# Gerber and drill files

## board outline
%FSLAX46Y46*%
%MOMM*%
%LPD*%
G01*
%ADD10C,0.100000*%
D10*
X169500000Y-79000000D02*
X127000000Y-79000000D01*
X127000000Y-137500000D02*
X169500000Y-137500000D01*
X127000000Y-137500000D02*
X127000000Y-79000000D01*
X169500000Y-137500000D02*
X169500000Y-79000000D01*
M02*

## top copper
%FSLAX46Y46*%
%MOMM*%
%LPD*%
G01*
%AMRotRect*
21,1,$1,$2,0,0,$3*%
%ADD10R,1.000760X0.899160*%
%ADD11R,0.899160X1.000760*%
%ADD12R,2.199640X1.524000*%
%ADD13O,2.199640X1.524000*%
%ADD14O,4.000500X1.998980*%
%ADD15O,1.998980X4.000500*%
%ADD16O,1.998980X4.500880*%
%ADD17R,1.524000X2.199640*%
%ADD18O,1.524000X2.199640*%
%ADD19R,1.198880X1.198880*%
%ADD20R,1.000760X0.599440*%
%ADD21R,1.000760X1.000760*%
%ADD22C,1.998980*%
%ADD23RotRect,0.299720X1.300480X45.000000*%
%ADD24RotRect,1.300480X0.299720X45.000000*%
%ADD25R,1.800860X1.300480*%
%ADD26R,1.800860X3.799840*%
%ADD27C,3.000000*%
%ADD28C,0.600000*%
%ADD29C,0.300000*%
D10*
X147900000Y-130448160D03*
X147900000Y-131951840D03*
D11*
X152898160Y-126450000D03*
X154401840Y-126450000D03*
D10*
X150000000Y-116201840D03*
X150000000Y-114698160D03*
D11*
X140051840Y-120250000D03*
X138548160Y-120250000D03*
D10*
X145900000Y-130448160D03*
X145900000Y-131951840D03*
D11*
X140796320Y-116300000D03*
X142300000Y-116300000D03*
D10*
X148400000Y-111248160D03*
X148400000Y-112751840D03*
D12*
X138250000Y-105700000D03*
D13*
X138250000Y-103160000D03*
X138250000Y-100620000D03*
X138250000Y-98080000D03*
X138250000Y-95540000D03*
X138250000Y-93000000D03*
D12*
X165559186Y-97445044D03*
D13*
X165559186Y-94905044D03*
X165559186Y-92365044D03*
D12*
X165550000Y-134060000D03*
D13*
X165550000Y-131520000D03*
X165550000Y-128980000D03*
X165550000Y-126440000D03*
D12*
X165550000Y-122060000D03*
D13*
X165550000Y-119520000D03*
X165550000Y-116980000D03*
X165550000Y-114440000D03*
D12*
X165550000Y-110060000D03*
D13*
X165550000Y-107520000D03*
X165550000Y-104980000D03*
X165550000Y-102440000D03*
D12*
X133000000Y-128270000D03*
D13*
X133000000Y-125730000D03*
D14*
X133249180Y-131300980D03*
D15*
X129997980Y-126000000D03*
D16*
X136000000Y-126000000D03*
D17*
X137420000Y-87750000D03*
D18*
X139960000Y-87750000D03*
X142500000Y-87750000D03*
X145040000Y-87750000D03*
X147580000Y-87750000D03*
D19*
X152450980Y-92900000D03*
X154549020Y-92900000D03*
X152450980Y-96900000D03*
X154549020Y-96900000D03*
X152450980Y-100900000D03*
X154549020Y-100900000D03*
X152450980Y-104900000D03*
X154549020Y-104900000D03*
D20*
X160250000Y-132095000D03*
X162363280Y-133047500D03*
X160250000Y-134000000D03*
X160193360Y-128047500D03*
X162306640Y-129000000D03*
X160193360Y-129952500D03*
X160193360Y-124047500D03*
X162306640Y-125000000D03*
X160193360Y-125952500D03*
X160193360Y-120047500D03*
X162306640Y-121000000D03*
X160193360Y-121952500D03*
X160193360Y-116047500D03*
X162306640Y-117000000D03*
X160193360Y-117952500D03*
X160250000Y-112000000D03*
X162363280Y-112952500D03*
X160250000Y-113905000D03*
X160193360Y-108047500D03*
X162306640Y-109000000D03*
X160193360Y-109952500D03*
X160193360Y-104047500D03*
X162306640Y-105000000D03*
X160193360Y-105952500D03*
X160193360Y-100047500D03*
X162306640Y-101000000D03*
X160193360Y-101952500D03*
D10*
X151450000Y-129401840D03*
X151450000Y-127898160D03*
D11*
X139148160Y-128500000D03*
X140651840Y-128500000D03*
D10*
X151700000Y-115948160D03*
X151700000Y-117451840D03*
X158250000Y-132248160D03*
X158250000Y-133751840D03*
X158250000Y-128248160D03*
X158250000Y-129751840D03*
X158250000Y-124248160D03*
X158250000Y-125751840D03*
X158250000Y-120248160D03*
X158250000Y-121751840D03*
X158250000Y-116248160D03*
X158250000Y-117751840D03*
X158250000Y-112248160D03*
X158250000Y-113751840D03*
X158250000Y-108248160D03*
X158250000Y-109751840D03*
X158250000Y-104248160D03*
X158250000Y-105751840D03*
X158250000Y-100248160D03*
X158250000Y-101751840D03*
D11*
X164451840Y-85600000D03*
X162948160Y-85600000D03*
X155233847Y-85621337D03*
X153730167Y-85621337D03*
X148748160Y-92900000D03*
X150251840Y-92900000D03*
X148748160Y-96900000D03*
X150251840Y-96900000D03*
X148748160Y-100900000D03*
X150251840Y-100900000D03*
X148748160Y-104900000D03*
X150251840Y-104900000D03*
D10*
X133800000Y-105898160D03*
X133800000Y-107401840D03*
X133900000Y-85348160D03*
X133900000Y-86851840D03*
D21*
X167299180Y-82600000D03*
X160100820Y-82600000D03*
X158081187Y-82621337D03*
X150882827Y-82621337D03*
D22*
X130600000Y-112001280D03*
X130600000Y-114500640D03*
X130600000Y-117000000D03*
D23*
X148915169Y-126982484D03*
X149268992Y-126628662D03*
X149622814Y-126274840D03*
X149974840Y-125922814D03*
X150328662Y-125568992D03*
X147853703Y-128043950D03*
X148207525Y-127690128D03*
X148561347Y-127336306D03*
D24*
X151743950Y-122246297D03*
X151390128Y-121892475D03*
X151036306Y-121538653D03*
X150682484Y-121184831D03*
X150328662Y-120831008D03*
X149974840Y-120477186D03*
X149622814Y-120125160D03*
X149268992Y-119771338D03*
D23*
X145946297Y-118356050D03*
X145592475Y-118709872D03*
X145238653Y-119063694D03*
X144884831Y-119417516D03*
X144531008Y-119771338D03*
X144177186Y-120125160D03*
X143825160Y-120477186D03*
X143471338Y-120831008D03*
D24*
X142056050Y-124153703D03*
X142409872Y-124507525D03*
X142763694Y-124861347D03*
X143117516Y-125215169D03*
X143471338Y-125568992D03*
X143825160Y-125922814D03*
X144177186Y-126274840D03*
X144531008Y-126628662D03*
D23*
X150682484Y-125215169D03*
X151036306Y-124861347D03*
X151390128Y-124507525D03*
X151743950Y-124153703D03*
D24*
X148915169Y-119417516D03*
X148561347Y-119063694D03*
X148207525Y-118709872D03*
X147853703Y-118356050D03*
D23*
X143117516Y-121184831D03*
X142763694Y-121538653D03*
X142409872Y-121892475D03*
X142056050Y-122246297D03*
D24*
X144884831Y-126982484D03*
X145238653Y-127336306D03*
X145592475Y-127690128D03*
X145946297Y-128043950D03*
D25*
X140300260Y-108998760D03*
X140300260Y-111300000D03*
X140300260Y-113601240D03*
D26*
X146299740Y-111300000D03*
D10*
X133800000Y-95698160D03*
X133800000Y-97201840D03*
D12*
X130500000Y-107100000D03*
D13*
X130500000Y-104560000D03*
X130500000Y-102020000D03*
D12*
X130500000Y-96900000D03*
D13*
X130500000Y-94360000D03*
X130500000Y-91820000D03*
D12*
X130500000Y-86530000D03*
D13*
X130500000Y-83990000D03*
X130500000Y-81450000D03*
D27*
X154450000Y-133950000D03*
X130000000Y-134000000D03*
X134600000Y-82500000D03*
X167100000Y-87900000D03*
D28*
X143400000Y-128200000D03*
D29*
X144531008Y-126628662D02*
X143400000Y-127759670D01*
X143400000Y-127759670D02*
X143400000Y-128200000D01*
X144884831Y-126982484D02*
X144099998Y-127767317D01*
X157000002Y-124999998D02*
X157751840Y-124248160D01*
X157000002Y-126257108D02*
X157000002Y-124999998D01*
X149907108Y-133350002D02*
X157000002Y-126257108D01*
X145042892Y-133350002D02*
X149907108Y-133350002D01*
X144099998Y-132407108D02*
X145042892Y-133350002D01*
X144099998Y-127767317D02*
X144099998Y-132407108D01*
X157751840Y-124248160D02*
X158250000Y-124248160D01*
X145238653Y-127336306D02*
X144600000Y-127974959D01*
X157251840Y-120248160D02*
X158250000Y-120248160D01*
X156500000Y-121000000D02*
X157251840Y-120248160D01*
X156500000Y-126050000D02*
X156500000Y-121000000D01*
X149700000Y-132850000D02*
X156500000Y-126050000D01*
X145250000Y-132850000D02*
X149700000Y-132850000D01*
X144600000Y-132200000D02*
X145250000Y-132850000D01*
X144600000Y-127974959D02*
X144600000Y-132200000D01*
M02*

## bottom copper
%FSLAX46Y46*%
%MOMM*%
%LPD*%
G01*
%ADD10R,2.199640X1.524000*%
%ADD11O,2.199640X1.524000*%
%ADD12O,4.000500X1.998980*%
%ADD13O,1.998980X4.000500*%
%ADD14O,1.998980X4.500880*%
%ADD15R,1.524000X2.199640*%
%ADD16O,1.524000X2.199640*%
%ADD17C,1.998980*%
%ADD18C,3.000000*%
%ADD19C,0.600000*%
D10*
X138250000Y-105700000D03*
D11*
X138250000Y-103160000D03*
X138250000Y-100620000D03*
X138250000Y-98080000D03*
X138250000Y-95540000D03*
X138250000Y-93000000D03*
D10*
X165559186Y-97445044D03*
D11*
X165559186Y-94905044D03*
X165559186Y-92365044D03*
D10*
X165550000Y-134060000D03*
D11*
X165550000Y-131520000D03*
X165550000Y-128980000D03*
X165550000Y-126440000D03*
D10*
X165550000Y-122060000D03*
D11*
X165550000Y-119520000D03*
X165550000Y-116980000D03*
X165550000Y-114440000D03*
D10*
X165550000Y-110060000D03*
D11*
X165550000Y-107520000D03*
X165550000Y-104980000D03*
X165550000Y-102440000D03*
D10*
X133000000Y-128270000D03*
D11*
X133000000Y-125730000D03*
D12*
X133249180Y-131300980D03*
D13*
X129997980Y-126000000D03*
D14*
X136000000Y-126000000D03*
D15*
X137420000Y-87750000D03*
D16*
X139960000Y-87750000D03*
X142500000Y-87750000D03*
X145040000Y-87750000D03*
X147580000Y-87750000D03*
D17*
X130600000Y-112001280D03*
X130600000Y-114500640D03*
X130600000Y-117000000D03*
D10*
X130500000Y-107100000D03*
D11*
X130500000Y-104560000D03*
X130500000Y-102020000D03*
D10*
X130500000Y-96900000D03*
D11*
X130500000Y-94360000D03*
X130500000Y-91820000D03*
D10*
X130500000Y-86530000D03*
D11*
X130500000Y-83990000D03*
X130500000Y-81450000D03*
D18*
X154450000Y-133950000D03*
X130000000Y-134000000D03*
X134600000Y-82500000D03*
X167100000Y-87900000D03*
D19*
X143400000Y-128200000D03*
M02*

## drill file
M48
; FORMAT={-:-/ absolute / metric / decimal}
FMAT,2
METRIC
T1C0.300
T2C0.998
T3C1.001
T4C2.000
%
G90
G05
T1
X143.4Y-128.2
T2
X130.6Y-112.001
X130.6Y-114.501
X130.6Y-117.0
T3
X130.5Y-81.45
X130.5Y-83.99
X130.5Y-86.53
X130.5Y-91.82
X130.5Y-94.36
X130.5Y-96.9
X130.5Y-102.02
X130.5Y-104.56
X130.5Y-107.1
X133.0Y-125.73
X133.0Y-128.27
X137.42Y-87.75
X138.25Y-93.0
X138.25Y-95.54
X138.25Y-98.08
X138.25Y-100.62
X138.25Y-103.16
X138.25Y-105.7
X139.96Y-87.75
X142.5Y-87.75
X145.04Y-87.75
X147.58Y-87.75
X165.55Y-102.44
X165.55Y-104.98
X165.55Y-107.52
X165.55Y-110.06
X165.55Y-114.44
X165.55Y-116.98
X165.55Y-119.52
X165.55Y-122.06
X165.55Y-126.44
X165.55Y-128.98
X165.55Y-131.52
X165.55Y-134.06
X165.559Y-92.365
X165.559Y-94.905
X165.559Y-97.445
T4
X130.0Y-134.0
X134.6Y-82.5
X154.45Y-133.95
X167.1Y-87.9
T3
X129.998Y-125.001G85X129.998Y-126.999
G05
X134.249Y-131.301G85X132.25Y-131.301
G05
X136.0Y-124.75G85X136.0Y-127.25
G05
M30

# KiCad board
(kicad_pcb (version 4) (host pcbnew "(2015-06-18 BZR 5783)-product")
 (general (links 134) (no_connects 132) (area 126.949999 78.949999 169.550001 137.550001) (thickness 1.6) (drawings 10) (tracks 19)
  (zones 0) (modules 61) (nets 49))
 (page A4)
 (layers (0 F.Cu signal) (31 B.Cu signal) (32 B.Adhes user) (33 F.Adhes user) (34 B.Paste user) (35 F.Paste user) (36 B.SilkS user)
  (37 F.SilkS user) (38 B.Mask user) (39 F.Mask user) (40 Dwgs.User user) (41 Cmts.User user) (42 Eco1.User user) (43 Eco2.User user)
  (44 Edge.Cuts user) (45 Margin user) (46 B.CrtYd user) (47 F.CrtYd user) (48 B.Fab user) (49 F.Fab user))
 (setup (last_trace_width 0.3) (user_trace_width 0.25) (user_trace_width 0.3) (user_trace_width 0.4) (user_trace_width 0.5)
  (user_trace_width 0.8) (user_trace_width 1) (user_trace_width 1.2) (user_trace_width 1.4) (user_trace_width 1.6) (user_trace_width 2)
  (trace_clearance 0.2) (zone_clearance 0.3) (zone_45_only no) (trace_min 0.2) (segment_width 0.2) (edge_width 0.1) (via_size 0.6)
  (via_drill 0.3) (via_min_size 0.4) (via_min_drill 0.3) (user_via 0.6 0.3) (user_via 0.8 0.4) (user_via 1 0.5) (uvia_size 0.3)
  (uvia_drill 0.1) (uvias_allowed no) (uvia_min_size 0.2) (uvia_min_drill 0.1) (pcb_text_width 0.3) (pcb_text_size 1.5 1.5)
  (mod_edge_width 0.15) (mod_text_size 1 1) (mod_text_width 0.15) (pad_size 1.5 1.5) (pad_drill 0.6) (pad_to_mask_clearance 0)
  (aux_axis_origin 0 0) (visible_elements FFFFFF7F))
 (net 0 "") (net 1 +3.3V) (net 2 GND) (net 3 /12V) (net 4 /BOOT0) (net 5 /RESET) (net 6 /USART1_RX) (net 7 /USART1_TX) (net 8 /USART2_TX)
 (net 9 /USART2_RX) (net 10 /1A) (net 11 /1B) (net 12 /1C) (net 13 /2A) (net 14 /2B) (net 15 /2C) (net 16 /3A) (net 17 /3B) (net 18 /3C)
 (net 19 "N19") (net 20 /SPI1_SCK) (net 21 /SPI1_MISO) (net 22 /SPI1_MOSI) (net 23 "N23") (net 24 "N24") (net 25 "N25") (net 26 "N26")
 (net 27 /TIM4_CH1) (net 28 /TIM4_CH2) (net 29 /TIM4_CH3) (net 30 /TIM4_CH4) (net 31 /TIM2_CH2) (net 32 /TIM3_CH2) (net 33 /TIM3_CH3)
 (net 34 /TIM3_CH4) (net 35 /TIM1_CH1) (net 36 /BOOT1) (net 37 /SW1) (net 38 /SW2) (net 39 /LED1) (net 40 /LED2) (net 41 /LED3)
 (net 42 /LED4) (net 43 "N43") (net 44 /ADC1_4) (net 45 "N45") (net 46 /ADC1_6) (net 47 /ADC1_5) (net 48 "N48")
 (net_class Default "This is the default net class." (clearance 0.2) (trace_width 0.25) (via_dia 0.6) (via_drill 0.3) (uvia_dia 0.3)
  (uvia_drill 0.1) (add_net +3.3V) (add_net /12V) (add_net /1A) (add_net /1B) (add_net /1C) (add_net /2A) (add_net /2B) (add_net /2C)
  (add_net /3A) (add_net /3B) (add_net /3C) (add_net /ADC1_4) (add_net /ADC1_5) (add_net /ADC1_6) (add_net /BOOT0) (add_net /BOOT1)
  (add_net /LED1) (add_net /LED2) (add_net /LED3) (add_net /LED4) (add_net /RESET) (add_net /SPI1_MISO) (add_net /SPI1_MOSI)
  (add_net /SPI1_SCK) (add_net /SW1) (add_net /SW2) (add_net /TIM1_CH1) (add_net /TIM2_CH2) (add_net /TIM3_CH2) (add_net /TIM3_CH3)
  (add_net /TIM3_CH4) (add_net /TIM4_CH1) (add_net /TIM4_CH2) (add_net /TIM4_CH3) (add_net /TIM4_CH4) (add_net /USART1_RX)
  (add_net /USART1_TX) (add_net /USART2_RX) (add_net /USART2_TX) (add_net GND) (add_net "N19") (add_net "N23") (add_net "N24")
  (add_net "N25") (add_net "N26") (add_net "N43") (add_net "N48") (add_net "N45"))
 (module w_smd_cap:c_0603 (layer F.Cu) (at 147.9 131.2 90)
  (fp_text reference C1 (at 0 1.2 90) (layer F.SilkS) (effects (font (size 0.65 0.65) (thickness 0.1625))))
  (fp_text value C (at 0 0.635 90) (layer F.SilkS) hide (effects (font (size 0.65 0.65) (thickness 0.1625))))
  (pad 1 smd rect (at 0.75184 0 90) (size 0.89916 1.00076) (layers F.Cu F.Paste F.Mask) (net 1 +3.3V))
  (pad 2 smd rect (at -0.75184 0 90) (size 0.89916 1.00076) (layers F.Cu F.Paste F.Mask) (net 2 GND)))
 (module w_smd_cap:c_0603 (layer F.Cu) (at 153.65 126.45 180)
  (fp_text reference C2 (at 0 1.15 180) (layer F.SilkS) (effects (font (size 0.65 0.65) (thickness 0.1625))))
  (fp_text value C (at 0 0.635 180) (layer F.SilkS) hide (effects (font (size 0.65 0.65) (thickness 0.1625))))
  (pad 1 smd rect (at 0.75184 0 180) (size 0.89916 1.00076) (layers F.Cu F.Paste F.Mask) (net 1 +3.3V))
  (pad 2 smd rect (at -0.75184 0 180) (size 0.89916 1.00076) (layers F.Cu F.Paste F.Mask) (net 2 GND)))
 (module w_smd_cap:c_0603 (layer F.Cu) (at 150 115.45 270)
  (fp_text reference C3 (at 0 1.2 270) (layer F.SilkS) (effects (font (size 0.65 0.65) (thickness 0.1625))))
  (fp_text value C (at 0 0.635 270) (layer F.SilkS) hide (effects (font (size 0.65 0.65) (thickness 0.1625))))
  (pad 1 smd rect (at 0.75184 0 270) (size 0.89916 1.00076) (layers F.Cu F.Paste F.Mask) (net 1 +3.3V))
  (pad 2 smd rect (at -0.75184 0 270) (size 0.89916 1.00076) (layers F.Cu F.Paste F.Mask) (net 2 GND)))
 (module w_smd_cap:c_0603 (layer F.Cu) (at 139.3 120.25)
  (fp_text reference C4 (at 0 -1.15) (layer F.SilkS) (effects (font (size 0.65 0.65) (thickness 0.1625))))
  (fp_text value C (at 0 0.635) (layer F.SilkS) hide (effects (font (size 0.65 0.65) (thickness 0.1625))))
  (pad 1 smd rect (at 0.75184 0) (size 0.89916 1.00076) (layers F.Cu F.Paste F.Mask) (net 1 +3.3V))
  (pad 2 smd rect (at -0.75184 0) (size 0.89916 1.00076) (layers F.Cu F.Paste F.Mask) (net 2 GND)))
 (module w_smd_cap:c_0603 (layer F.Cu) (at 145.9 131.2 90)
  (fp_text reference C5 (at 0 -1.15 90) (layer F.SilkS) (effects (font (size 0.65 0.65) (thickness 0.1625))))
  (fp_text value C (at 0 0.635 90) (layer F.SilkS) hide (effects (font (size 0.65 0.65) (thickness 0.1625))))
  (pad 1 smd rect (at 0.75184 0 90) (size 0.89916 1.00076) (layers F.Cu F.Paste F.Mask) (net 1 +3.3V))
  (pad 2 smd rect (at -0.75184 0 90) (size 0.89916 1.00076) (layers F.Cu F.Paste F.Mask) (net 2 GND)))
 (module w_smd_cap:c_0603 (layer F.Cu) (at 141.54816 116.3 180)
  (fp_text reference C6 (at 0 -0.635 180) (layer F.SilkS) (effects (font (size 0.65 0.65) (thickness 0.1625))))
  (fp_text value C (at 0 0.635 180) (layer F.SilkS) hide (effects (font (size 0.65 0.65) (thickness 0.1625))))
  (pad 1 smd rect (at 0.75184 0 180) (size 0.89916 1.00076) (layers F.Cu F.Paste F.Mask) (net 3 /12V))
  (pad 2 smd rect (at -0.75184 0 180) (size 0.89916 1.00076) (layers F.Cu F.Paste F.Mask) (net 2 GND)))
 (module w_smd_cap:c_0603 (layer F.Cu) (at 148.4 112 90)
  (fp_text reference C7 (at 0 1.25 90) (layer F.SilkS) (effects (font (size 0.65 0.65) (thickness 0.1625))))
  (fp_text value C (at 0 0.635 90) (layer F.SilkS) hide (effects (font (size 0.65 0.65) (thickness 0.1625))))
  (pad 1 smd rect (at 0.75184 0 90) (size 0.89916 1.00076) (layers F.Cu F.Paste F.Mask) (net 1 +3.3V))
  (pad 2 smd rect (at -0.75184 0 90) (size 0.89916 1.00076) (layers F.Cu F.Paste F.Mask) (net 2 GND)))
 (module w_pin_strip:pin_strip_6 (layer F.Cu) (at 138.25 99.35 90)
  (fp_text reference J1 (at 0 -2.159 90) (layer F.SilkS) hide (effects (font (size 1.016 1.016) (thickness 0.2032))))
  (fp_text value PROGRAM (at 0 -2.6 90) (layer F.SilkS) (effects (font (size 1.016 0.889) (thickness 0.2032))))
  (pad 1 thru_hole rect (at -6.35 0 90) (size 1.524 2.19964) (drill 1.00076) (layers *.Cu *.Mask F.SilkS) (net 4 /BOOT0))
  (pad 2 thru_hole oval (at -3.81 0 90) (size 1.524 2.19964) (drill 1.00076) (layers *.Cu *.Mask F.SilkS) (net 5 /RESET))
  (pad 3 thru_hole oval (at -1.27 0 90) (size 1.524 2.19964) (drill 1.00076) (layers *.Cu *.Mask F.SilkS) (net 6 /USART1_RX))
  (pad 4 thru_hole oval (at 1.27 0 90) (size 1.524 2.19964) (drill 1.00076) (layers *.Cu *.Mask F.SilkS) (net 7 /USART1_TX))
  (pad 5 thru_hole oval (at 3.81 0 90) (size 1.524 2.19964) (drill 1.00076) (layers *.Cu *.Mask F.SilkS) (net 2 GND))
  (pad 6 thru_hole oval (at 6.35 0 90) (size 1.524 2.19964) (drill 1.00076) (layers *.Cu *.Mask F.SilkS) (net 1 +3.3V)))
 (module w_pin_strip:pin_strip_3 (layer F.Cu) (at 165.559186 94.905044 90)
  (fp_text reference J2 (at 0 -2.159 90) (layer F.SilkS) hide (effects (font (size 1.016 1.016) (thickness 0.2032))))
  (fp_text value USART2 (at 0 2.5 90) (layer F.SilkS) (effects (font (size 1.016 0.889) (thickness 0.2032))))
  (pad 1 thru_hole rect (at -2.54 0 90) (size 1.524 2.19964) (drill 1.00076) (layers *.Cu *.Mask F.SilkS) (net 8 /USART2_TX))
  (pad 2 thru_hole oval (at 0 0 90) (size 1.524 2.19964) (drill 1.00076) (layers *.Cu *.Mask F.SilkS) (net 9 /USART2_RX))
  (pad 3 thru_hole oval (at 2.54 0 90) (size 1.524 2.19964) (drill 1.00076) (layers *.Cu *.Mask F.SilkS) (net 2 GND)))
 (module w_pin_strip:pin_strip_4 (layer F.Cu) (at 165.55 130.25 90)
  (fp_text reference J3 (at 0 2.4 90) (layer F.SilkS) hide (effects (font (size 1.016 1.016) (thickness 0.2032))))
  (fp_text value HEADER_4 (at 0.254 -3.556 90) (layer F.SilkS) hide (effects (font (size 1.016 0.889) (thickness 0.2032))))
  (pad 1 thru_hole rect (at -3.81 0 90) (size 1.524 2.19964) (drill 1.00076) (layers *.Cu *.Mask F.SilkS) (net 3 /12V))
  (pad 2 thru_hole oval (at -1.27 0 90) (size 1.524 2.19964) (drill 1.00076) (layers *.Cu *.Mask F.SilkS) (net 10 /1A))
  (pad 3 thru_hole oval (at 1.27 0 90) (size 1.524 2.19964) (drill 1.00076) (layers *.Cu *.Mask F.SilkS) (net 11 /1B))
  (pad 4 thru_hole oval (at 3.81 0 90) (size 1.524 2.19964) (drill 1.00076) (layers *.Cu *.Mask F.SilkS) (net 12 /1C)))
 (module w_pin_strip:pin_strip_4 (layer F.Cu) (at 165.55 118.25 90)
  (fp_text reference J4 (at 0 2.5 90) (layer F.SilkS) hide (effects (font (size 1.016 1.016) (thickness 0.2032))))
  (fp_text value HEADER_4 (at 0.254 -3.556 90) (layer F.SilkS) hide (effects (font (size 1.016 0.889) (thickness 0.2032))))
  (pad 1 thru_hole rect (at -3.81 0 90) (size 1.524 2.19964) (drill 1.00076) (layers *.Cu *.Mask F.SilkS) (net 3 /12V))
  (pad 2 thru_hole oval (at -1.27 0 90) (size 1.524 2.19964) (drill 1.00076) (layers *.Cu *.Mask F.SilkS) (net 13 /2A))
  (pad 3 thru_hole oval (at 1.27 0 90) (size 1.524 2.19964) (drill 1.00076) (layers *.Cu *.Mask F.SilkS) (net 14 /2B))
  (pad 4 thru_hole oval (at 3.81 0 90) (size 1.524 2.19964) (drill 1.00076) (layers *.Cu *.Mask F.SilkS) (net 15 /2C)))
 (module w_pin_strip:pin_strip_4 (layer F.Cu) (at 165.55 106.25 90)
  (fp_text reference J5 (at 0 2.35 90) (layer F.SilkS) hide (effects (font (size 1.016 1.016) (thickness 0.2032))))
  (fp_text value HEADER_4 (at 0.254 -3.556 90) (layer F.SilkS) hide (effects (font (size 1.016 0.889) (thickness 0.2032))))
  (pad 1 thru_hole rect (at -3.81 0 90) (size 1.524 2.19964) (drill 1.00076) (layers *.Cu *.Mask F.SilkS) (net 3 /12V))
  (pad 2 thru_hole oval (at -1.27 0 90) (size 1.524 2.19964) (drill 1.00076) (layers *.Cu *.Mask F.SilkS) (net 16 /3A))
  (pad 3 thru_hole oval (at 1.27 0 90) (size 1.524 2.19964) (drill 1.00076) (layers *.Cu *.Mask F.SilkS) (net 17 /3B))
  (pad 4 thru_hole oval (at 3.81 0 90) (size 1.524 2.19964) (drill 1.00076) (layers *.Cu *.Mask F.SilkS) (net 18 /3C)))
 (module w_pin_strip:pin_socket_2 (layer F.Cu) (at 133 127 90)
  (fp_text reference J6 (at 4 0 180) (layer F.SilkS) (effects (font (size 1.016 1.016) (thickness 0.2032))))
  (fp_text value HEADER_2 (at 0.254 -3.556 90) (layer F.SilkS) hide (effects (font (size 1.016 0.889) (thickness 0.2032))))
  (pad 1 thru_hole rect (at -1.27 0 90) (size 1.524 2.19964) (drill 1.00076) (layers *.Cu *.Mask F.SilkS) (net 3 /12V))
  (pad 2 thru_hole oval (at 1.27 0 90) (size 1.524 2.19964) (drill 1.00076) (layers *.Cu *.Mask F.SilkS) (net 2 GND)))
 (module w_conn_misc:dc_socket (layer F.Cu) (at 129.74906 126 270)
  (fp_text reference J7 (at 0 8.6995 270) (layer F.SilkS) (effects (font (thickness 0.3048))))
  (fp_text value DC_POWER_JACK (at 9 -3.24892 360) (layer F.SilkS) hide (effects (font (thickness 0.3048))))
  (pad 1 thru_hole oval (at 5.30098 -3.50012 270) (size 1.99898 4.0005) (drill oval 1.00076 2.99974) (layers *.Cu *.Mask F.SilkS)
   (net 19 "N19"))
  (pad 2 thru_hole oval (at 0 -0.24892 270) (size 4.0005 1.99898) (drill oval 2.99974 1.00076) (layers *.Cu *.Mask F.SilkS) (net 2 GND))
  (pad 3 thru_hole oval (at 0 -6.25094 270) (size 4.50088 1.99898) (drill oval 3.50012 1.00076) (layers *.Cu *.Mask F.SilkS) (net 2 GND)))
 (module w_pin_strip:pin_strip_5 (layer F.Cu) (at 142.5 87.75)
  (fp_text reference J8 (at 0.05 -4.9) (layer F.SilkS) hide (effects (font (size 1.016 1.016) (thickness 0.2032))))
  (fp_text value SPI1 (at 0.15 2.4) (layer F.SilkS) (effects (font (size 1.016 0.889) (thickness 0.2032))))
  (pad 1 thru_hole rect (at -5.08 0) (size 1.524 2.19964) (drill 1.00076) (layers *.Cu *.Mask F.SilkS) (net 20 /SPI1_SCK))
  (pad 2 thru_hole oval (at -2.54 0) (size 1.524 2.19964) (drill 1.00076) (layers *.Cu *.Mask F.SilkS) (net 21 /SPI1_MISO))
  (pad 3 thru_hole oval (at 0 0) (size 1.524 2.19964) (drill 1.00076) (layers *.Cu *.Mask F.SilkS) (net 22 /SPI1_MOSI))
  (pad 4 thru_hole oval (at 2.54 0) (size 1.524 2.19964) (drill 1.00076) (layers *.Cu *.Mask F.SilkS) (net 2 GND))
  (pad 5 thru_hole oval (at 5.08 0) (size 1.524 2.19964) (drill 1.00076) (layers *.Cu *.Mask F.SilkS) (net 1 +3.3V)))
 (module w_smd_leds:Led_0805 (layer F.Cu) (at 153.5 92.9)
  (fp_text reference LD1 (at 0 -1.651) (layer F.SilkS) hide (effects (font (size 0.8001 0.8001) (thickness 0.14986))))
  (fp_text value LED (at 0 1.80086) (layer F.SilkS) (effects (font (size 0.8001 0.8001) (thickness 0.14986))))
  (pad 1 smd rect (at -1.04902 0) (size 1.19888 1.19888) (layers F.Cu F.Paste F.Mask) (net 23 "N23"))
  (pad 2 smd rect (at 1.04902 0) (size 1.19888 1.19888) (layers F.Cu F.Paste F.Mask) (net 2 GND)))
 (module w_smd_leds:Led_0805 (layer F.Cu) (at 153.5 96.9)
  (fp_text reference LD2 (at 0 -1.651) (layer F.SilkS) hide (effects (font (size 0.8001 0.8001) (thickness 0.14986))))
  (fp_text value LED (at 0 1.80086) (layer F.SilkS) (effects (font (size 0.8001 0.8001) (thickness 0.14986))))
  (pad 1 smd rect (at -1.04902 0) (size 1.19888 1.19888) (layers F.Cu F.Paste F.Mask) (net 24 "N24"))
  (pad 2 smd rect (at 1.04902 0) (size 1.19888 1.19888) (layers F.Cu F.Paste F.Mask) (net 2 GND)))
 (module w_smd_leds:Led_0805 (layer F.Cu) (at 153.5 100.9)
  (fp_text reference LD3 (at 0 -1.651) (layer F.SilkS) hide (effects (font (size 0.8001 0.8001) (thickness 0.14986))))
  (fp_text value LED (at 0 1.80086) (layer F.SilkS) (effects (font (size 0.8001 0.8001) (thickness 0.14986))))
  (pad 1 smd rect (at -1.04902 0) (size 1.19888 1.19888) (layers F.Cu F.Paste F.Mask) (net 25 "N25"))
  (pad 2 smd rect (at 1.04902 0) (size 1.19888 1.19888) (layers F.Cu F.Paste F.Mask) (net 2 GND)))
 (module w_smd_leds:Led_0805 (layer F.Cu) (at 153.5 104.9)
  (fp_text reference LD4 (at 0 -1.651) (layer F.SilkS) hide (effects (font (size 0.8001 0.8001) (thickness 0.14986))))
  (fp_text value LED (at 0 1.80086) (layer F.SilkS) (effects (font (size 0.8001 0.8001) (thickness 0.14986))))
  (pad 1 smd rect (at -1.04902 0) (size 1.19888 1.19888) (layers F.Cu F.Paste F.Mask) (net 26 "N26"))
  (pad 2 smd rect (at 1.04902 0) (size 1.19888 1.19888) (layers F.Cu F.Paste F.Mask) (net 2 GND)))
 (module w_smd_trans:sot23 (layer F.Cu) (at 161.30664 133.0475 270)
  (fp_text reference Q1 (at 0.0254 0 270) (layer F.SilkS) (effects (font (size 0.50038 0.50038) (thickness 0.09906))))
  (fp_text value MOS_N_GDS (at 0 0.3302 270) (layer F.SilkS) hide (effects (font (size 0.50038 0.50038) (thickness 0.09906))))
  (pad 1 smd rect (at -0.9525 1.05664 270) (size 0.59944 1.00076) (layers F.Cu F.Paste F.Mask) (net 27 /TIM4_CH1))
  (pad 2 smd rect (at 0 -1.05664 270) (size 0.59944 1.00076) (layers F.Cu F.Paste F.Mask) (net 10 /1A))
  (pad 3 smd rect (at 0.9525 1.05664 270) (size 0.59944 1.00076) (layers F.Cu F.Paste F.Mask) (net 2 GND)))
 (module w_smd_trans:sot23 (layer F.Cu) (at 161.25 129 270)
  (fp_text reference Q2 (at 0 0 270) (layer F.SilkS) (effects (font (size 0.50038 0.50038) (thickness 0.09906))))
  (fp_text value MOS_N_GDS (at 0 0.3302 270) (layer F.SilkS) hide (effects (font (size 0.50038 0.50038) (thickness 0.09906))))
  (pad 1 smd rect (at -0.9525 1.05664 270) (size 0.59944 1.00076) (layers F.Cu F.Paste F.Mask) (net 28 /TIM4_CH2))
  (pad 2 smd rect (at 0 -1.05664 270) (size 0.59944 1.00076) (layers F.Cu F.Paste F.Mask) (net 11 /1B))
  (pad 3 smd rect (at 0.9525 1.05664 270) (size 0.59944 1.00076) (layers F.Cu F.Paste F.Mask) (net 2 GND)))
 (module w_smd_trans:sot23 (layer F.Cu) (at 161.25 125 270)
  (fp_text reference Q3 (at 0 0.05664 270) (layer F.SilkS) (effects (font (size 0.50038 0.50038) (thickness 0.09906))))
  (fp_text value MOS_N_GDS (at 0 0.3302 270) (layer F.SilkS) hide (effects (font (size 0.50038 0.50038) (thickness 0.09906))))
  (pad 1 smd rect (at -0.9525 1.05664 270) (size 0.59944 1.00076) (layers F.Cu F.Paste F.Mask) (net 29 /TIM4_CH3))
  (pad 2 smd rect (at 0 -1.05664 270) (size 0.59944 1.00076) (layers F.Cu F.Paste F.Mask) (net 12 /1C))
  (pad 3 smd rect (at 0.9525 1.05664 270) (size 0.59944 1.00076) (layers F.Cu F.Paste F.Mask) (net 2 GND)))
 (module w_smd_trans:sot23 (layer F.Cu) (at 161.25 121 270)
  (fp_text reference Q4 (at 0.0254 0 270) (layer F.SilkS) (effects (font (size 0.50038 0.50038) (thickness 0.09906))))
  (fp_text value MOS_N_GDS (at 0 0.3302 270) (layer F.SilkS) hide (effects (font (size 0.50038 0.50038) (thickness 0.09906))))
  (pad 1 smd rect (at -0.9525 1.05664 270) (size 0.59944 1.00076) (layers F.Cu F.Paste F.Mask) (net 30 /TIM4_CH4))
  (pad 2 smd rect (at 0 -1.05664 270) (size 0.59944 1.00076) (layers F.Cu F.Paste F.Mask) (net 13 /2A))
  (pad 3 smd rect (at 0.9525 1.05664 270) (size 0.59944 1.00076) (layers F.Cu F.Paste F.Mask) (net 2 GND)))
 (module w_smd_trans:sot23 (layer F.Cu) (at 161.25 117 270)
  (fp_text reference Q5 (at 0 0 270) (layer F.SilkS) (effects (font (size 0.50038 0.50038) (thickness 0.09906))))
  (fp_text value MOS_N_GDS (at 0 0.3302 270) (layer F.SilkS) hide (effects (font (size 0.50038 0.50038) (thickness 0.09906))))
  (pad 1 smd rect (at -0.9525 1.05664 270) (size 0.59944 1.00076) (layers F.Cu F.Paste F.Mask) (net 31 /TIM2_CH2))
  (pad 2 smd rect (at 0 -1.05664 270) (size 0.59944 1.00076) (layers F.Cu F.Paste F.Mask) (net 14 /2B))
  (pad 3 smd rect (at 0.9525 1.05664 270) (size 0.59944 1.00076) (layers F.Cu F.Paste F.Mask) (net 2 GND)))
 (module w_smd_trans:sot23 (layer F.Cu) (at 161.30664 112.9525 270)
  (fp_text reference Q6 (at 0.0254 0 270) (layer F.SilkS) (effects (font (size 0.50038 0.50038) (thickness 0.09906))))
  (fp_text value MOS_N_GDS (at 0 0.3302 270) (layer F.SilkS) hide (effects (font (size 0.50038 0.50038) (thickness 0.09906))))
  (pad 1 smd rect (at -0.9525 1.05664 270) (size 0.59944 1.00076) (layers F.Cu F.Paste F.Mask) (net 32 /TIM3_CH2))
  (pad 2 smd rect (at 0 -1.05664 270) (size 0.59944 1.00076) (layers F.Cu F.Paste F.Mask) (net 15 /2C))
  (pad 3 smd rect (at 0.9525 1.05664 270) (size 0.59944 1.00076) (layers F.Cu F.Paste F.Mask) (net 2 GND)))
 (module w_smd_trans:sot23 (layer F.Cu) (at 161.25 109 270)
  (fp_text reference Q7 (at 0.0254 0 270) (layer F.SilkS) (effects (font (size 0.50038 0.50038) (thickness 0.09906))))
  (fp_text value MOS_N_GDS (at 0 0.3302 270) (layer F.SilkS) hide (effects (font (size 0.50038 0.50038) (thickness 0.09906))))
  (pad 1 smd rect (at -0.9525 1.05664 270) (size 0.59944 1.00076) (layers F.Cu F.Paste F.Mask) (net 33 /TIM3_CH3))
  (pad 2 smd rect (at 0 -1.05664 270) (size 0.59944 1.00076) (layers F.Cu F.Paste F.Mask) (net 16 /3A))
  (pad 3 smd rect (at 0.9525 1.05664 270) (size 0.59944 1.00076) (layers F.Cu F.Paste F.Mask) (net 2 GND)))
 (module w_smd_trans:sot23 (layer F.Cu) (at 161.25 105 270)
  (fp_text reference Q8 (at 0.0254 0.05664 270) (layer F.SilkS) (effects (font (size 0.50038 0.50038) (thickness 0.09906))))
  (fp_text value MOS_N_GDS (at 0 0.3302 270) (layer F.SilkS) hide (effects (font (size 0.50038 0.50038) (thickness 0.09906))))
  (pad 1 smd rect (at -0.9525 1.05664 270) (size 0.59944 1.00076) (layers F.Cu F.Paste F.Mask) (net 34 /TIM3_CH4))
  (pad 2 smd rect (at 0 -1.05664 270) (size 0.59944 1.00076) (layers F.Cu F.Paste F.Mask) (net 17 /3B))
  (pad 3 smd rect (at 0.9525 1.05664 270) (size 0.59944 1.00076) (layers F.Cu F.Paste F.Mask) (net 2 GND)))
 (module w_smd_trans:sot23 (layer F.Cu) (at 161.25 101 270)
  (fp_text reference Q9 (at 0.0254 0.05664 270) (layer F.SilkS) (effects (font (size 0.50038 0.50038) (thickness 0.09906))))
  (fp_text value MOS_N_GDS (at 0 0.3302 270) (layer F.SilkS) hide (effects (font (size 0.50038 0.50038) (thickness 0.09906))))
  (pad 1 smd rect (at -0.9525 1.05664 270) (size 0.59944 1.00076) (layers F.Cu F.Paste F.Mask) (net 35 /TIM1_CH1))
  (pad 2 smd rect (at 0 -1.05664 270) (size 0.59944 1.00076) (layers F.Cu F.Paste F.Mask) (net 18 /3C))
  (pad 3 smd rect (at 0.9525 1.05664 270) (size 0.59944 1.00076) (layers F.Cu F.Paste F.Mask) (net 2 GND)))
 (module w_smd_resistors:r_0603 (layer F.Cu) (at 151.45 128.65 270)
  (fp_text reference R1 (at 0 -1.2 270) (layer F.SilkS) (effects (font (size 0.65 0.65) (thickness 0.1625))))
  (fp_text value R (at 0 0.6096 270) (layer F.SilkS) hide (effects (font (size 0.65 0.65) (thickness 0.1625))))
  (pad 1 smd rect (at 0.75184 0 270) (size 0.89916 1.00076) (layers F.Cu F.Paste F.Mask) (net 1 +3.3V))
  (pad 2 smd rect (at -0.75184 0 270) (size 0.89916 1.00076) (layers F.Cu F.Paste F.Mask) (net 5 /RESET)))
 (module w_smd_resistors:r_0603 (layer F.Cu) (at 139.9 128.5 180)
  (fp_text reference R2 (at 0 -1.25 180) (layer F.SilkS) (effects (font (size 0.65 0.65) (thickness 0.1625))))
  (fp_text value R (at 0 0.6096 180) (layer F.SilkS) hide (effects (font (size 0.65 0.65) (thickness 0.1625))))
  (pad 1 smd rect (at 0.75184 0 180) (size 0.89916 1.00076) (layers F.Cu F.Paste F.Mask) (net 2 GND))
  (pad 2 smd rect (at -0.75184 0 180) (size 0.89916 1.00076) (layers F.Cu F.Paste F.Mask) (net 4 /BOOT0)))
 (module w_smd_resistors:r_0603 (layer F.Cu) (at 151.7 116.7 90)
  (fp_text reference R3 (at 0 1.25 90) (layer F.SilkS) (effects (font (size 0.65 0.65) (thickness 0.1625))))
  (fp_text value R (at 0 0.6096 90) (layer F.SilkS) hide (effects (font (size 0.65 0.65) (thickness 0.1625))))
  (pad 1 smd rect (at 0.75184 0 90) (size 0.89916 1.00076) (layers F.Cu F.Paste F.Mask) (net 2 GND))
  (pad 2 smd rect (at -0.75184 0 90) (size 0.89916 1.00076) (layers F.Cu F.Paste F.Mask) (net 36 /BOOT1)))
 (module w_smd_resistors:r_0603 (layer F.Cu) (at 158.25 133 90)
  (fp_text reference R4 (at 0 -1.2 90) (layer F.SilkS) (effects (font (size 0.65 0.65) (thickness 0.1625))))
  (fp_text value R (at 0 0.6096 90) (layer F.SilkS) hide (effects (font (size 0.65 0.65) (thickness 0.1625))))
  (pad 1 smd rect (at 0.75184 0 90) (size 0.89916 1.00076) (layers F.Cu F.Paste F.Mask) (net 27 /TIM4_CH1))
  (pad 2 smd rect (at -0.75184 0 90) (size 0.89916 1.00076) (layers F.Cu F.Paste F.Mask) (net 2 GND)))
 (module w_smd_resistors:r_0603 (layer F.Cu) (at 158.25 129 90)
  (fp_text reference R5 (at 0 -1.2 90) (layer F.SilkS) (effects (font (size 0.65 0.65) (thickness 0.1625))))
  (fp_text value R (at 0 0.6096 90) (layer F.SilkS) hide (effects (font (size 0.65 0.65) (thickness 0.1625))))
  (pad 1 smd rect (at 0.75184 0 90) (size 0.89916 1.00076) (layers F.Cu F.Paste F.Mask) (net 28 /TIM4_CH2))
  (pad 2 smd rect (at -0.75184 0 90) (size 0.89916 1.00076) (layers F.Cu F.Paste F.Mask) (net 2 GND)))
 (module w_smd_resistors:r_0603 (layer F.Cu) (at 158.25 125 90)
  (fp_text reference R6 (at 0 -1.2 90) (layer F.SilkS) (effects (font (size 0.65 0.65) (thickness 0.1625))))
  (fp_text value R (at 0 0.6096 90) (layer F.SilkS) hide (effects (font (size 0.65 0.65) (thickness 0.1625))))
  (pad 1 smd rect (at 0.75184 0 90) (size 0.89916 1.00076) (layers F.Cu F.Paste F.Mask) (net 29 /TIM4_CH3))
  (pad 2 smd rect (at -0.75184 0 90) (size 0.89916 1.00076) (layers F.Cu F.Paste F.Mask) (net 2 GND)))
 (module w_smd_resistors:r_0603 (layer F.Cu) (at 158.25 121 90)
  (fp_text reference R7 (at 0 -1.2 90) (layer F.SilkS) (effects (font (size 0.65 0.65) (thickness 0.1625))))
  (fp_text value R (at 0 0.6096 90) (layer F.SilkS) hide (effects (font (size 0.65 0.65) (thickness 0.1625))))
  (pad 1 smd rect (at 0.75184 0 90) (size 0.89916 1.00076) (layers F.Cu F.Paste F.Mask) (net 30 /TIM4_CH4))
  (pad 2 smd rect (at -0.75184 0 90) (size 0.89916 1.00076) (layers F.Cu F.Paste F.Mask) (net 2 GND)))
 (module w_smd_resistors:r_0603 (layer F.Cu) (at 158.25 117 90)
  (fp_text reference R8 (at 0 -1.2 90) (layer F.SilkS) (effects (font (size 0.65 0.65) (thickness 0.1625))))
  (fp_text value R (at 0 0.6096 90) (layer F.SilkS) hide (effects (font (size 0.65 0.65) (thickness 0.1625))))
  (pad 1 smd rect (at 0.75184 0 90) (size 0.89916 1.00076) (layers F.Cu F.Paste F.Mask) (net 31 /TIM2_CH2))
  (pad 2 smd rect (at -0.75184 0 90) (size 0.89916 1.00076) (layers F.Cu F.Paste F.Mask) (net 2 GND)))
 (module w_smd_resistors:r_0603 (layer F.Cu) (at 158.25 113 90)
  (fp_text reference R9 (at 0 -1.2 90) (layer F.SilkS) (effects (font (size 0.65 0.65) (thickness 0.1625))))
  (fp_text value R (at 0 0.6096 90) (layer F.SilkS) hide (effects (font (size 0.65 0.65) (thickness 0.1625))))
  (pad 1 smd rect (at 0.75184 0 90) (size 0.89916 1.00076) (layers F.Cu F.Paste F.Mask) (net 32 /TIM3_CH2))
  (pad 2 smd rect (at -0.75184 0 90) (size 0.89916 1.00076) (layers F.Cu F.Paste F.Mask) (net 2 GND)))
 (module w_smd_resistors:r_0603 (layer F.Cu) (at 158.25 109 90)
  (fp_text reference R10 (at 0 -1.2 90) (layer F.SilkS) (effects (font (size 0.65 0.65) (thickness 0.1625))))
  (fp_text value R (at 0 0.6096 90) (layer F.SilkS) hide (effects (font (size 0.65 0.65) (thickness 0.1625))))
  (pad 1 smd rect (at 0.75184 0 90) (size 0.89916 1.00076) (layers F.Cu F.Paste F.Mask) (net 33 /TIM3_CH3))
  (pad 2 smd rect (at -0.75184 0 90) (size 0.89916 1.00076) (layers F.Cu F.Paste F.Mask) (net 2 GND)))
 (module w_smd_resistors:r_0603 (layer F.Cu) (at 158.25 105 90)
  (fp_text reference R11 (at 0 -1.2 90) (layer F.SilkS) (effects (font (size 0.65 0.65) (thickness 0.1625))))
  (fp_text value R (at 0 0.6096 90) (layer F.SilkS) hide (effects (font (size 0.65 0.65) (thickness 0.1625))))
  (pad 1 smd rect (at 0.75184 0 90) (size 0.89916 1.00076) (layers F.Cu F.Paste F.Mask) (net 34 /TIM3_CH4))
  (pad 2 smd rect (at -0.75184 0 90) (size 0.89916 1.00076) (layers F.Cu F.Paste F.Mask) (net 2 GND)))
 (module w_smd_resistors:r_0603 (layer F.Cu) (at 158.25 101 90)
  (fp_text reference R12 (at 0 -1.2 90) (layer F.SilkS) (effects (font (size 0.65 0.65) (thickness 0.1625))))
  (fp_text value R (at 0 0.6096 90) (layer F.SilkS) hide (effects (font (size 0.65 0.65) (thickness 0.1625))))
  (pad 1 smd rect (at 0.75184 0 90) (size 0.89916 1.00076) (layers F.Cu F.Paste F.Mask) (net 35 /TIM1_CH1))
  (pad 2 smd rect (at -0.75184 0 90) (size 0.89916 1.00076) (layers F.Cu F.Paste F.Mask) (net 2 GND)))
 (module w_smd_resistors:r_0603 (layer F.Cu) (at 163.7 85.6)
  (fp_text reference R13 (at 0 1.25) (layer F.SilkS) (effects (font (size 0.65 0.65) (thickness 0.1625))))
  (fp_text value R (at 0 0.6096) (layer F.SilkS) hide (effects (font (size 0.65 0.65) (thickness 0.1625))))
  (pad 1 smd rect (at 0.75184 0) (size 0.89916 1.00076) (layers F.Cu F.Paste F.Mask) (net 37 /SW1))
  (pad 2 smd rect (at -0.75184 0) (size 0.89916 1.00076) (layers F.Cu F.Paste F.Mask) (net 2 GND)))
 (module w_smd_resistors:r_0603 (layer F.Cu) (at 154.482007 85.621337)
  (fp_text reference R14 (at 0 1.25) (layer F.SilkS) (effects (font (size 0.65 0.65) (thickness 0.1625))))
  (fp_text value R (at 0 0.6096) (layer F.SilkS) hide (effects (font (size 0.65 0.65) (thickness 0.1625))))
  (pad 1 smd rect (at 0.75184 0) (size 0.89916 1.00076) (layers F.Cu F.Paste F.Mask) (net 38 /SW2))
  (pad 2 smd rect (at -0.75184 0) (size 0.89916 1.00076) (layers F.Cu F.Paste F.Mask) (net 2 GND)))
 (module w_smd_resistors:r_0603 (layer F.Cu) (at 149.5 92.9 180)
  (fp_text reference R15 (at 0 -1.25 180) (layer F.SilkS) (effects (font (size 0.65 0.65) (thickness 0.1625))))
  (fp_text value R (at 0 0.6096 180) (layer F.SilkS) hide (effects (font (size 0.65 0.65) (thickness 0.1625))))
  (pad 1 smd rect (at 0.75184 0 180) (size 0.89916 1.00076) (layers F.Cu F.Paste F.Mask) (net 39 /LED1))
  (pad 2 smd rect (at -0.75184 0 180) (size 0.89916 1.00076) (layers F.Cu F.Paste F.Mask) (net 23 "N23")))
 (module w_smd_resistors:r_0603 (layer F.Cu) (at 149.5 96.9 180)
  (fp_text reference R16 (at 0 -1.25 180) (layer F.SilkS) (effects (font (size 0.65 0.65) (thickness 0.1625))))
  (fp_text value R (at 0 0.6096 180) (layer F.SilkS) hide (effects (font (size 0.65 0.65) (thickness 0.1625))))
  (pad 1 smd rect (at 0.75184 0 180) (size 0.89916 1.00076) (layers F.Cu F.Paste F.Mask) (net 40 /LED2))
  (pad 2 smd rect (at -0.75184 0 180) (size 0.89916 1.00076) (layers F.Cu F.Paste F.Mask) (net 24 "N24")))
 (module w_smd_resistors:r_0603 (layer F.Cu) (at 149.5 100.9 180)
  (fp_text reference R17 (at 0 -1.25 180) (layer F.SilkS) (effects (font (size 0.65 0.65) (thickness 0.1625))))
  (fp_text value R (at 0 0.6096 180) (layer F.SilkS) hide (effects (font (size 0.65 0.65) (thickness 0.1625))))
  (pad 1 smd rect (at 0.75184 0 180) (size 0.89916 1.00076) (layers F.Cu F.Paste F.Mask) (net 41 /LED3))
  (pad 2 smd rect (at -0.75184 0 180) (size 0.89916 1.00076) (layers F.Cu F.Paste F.Mask) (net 25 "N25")))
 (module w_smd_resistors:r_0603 (layer F.Cu) (at 149.5 104.9 180)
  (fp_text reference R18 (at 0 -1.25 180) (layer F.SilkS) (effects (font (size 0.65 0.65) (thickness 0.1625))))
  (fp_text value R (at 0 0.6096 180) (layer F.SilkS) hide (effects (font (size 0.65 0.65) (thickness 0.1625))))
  (pad 1 smd rect (at 0.75184 0 180) (size 0.89916 1.00076) (layers F.Cu F.Paste F.Mask) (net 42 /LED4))
  (pad 2 smd rect (at -0.75184 0 180) (size 0.89916 1.00076) (layers F.Cu F.Paste F.Mask) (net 26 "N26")))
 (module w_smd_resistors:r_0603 (layer F.Cu) (at 133.8 106.65 90)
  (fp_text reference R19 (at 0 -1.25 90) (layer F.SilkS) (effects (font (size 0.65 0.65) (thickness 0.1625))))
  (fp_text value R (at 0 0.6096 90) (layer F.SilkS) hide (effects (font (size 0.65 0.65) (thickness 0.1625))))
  (pad 1 smd rect (at 0.75184 0 90) (size 0.89916 1.00076) (layers F.Cu F.Paste F.Mask) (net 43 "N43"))
  (pad 2 smd rect (at -0.75184 0 90) (size 0.89916 1.00076) (layers F.Cu F.Paste F.Mask) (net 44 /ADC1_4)))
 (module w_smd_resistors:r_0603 (layer F.Cu) (at 133.9 86.1 90)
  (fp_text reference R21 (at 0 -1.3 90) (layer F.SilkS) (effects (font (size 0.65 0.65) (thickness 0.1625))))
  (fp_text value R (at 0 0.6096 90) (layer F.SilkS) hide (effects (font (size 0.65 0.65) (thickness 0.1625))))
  (pad 1 smd rect (at 0.75184 0 90) (size 0.89916 1.00076) (layers F.Cu F.Paste F.Mask) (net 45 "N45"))
  (pad 2 smd rect (at -0.75184 0 90) (size 0.89916 1.00076) (layers F.Cu F.Paste F.Mask) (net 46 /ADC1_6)))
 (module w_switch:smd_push (layer F.Cu) (at 163.7 82.6 180) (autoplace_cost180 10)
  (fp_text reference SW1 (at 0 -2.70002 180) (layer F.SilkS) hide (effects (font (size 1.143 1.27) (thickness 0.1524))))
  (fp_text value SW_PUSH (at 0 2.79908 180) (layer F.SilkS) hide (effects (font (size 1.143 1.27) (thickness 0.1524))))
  (pad 1 smd rect (at -3.59918 0 180) (size 1.00076 1.00076) (layers F.Cu F.Paste F.Mask) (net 37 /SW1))
  (pad 2 smd rect (at 3.59918 0 180) (size 1.00076 1.00076) (layers F.Cu F.Paste F.Mask) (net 1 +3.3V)))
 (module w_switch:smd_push (layer F.Cu) (at 154.482007 82.621337 180) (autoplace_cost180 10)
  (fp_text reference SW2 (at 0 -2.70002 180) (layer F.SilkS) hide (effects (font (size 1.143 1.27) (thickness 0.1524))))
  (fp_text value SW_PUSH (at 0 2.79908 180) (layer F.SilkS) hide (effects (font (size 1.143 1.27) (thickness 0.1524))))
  (pad 1 smd rect (at -3.59918 0 180) (size 1.00076 1.00076) (layers F.Cu F.Paste F.Mask) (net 1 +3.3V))
  (pad 2 smd rect (at 3.59918 0 180) (size 1.00076 1.00076) (layers F.Cu F.Paste F.Mask) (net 38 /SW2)))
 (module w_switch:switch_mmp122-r (layer F.Cu) (at 130.6 114.50064 270)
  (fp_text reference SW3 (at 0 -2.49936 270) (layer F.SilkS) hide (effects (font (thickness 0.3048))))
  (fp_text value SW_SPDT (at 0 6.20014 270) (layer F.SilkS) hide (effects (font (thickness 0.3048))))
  (pad 1 thru_hole circle (at -2.49936 0 270) (size 1.99898 1.99898) (drill 0.99822) (layers *.Cu *.Mask F.SilkS) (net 19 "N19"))
  (pad 2 thru_hole circle (at 0 0 270) (size 1.99898 1.99898) (drill 0.99822) (layers *.Cu *.Mask F.SilkS) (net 3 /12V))
  (pad 3 thru_hole circle (at 2.49936 0 270) (size 1.99898 1.99898) (drill 0.99822) (layers *.Cu *.Mask F.SilkS)))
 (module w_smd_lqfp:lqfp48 (layer F.Cu) (at 146.9 123.2 45)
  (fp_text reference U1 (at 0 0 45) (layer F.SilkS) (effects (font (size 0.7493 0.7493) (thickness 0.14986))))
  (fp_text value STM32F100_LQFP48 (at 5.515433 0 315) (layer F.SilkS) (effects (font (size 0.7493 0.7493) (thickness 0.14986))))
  (pad 4 smd rect (at -1.24968 4.09956 45) (size 0.29972 1.30048) (layers F.Cu F.Paste F.Mask))
  (pad 5 smd rect (at -0.7493 4.09956 45) (size 0.29972 1.30048) (layers F.Cu F.Paste F.Mask))
  (pad 6 smd rect (at -0.24892 4.09956 45) (size 0.29972 1.30048) (layers F.Cu F.Paste F.Mask))
  (pad 7 smd rect (at 0.24892 4.09956 45) (size 0.29972 1.30048) (layers F.Cu F.Paste F.Mask) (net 5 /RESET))
  (pad 8 smd rect (at 0.7493 4.09956 45) (size 0.29972 1.30048) (layers F.Cu F.Paste F.Mask) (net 2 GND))
  (pad 1 smd rect (at -2.75082 4.09956 45) (size 0.29972 1.30048) (layers F.Cu F.Paste F.Mask) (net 1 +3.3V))
  (pad 2 smd rect (at -2.25044 4.09956 45) (size 0.29972 1.30048) (layers F.Cu F.Paste F.Mask))
  (pad 3 smd rect (at -1.75006 4.09956 45) (size 0.29972 1.30048) (layers F.Cu F.Paste F.Mask))
  (pad 13 smd rect (at 4.09956 2.75082 45) (size 1.30048 0.29972) (layers F.Cu F.Paste F.Mask) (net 9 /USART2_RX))
  (pad 14 smd rect (at 4.09956 2.25044 45) (size 1.30048 0.29972) (layers F.Cu F.Paste F.Mask) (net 44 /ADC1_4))
  (pad 15 smd rect (at 4.09956 1.75006 45) (size 1.30048 0.29972) (layers F.Cu F.Paste F.Mask) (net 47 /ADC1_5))
  (pad 16 smd rect (at 4.09956 1.24968 45) (size 1.30048 0.29972) (layers F.Cu F.Paste F.Mask) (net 46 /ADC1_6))
  (pad 17 smd rect (at 4.09956 0.7493 45) (size 1.30048 0.29972) (layers F.Cu F.Paste F.Mask) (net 32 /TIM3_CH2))
  (pad 18 smd rect (at 4.09956 0.24892 45) (size 1.30048 0.29972) (layers F.Cu F.Paste F.Mask) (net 33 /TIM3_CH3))
  (pad 19 smd rect (at 4.09956 -0.24892 45) (size 1.30048 0.29972) (layers F.Cu F.Paste F.Mask) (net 34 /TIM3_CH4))
  (pad 20 smd rect (at 4.09956 -0.7493 45) (size 1.30048 0.29972) (layers F.Cu F.Paste F.Mask) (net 36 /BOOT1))
  (pad 25 smd rect (at 2.75082 -4.09956 45) (size 0.29972 1.30048) (layers F.Cu F.Paste F.Mask) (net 42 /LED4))
  (pad 26 smd rect (at 2.25044 -4.09956 45) (size 0.29972 1.30048) (layers F.Cu F.Paste F.Mask) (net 20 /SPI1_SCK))
  (pad 27 smd rect (at 1.75006 -4.09956 45) (size 0.29972 1.30048) (layers F.Cu F.Paste F.Mask) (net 21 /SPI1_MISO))
  (pad 28 smd rect (at 1.24968 -4.09956 45) (size 0.29972 1.30048) (layers F.Cu F.Paste F.Mask) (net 22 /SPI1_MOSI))
  (pad 29 smd rect (at 0.7493 -4.09956 45) (size 0.29972 1.30048) (layers F.Cu F.Paste F.Mask) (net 35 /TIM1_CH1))
  (pad 30 smd rect (at 0.24892 -4.09956 45) (size 0.29972 1.30048) (layers F.Cu F.Paste F.Mask) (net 7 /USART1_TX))
  (pad 31 smd rect (at -0.24892 -4.09956 45) (size 0.29972 1.30048) (layers F.Cu F.Paste F.Mask) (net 6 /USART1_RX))
  (pad 32 smd rect (at -0.7493 -4.09956 45) (size 0.29972 1.30048) (layers F.Cu F.Paste F.Mask) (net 37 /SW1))
  (pad 37 smd rect (at -4.09956 -2.75082 45) (size 1.30048 0.29972) (layers F.Cu F.Paste F.Mask))
  (pad 38 smd rect (at -4.09956 -2.25044 45) (size 1.30048 0.29972) (layers F.Cu F.Paste F.Mask))
  (pad 39 smd rect (at -4.09956 -1.75006 45) (size 1.30048 0.29972) (layers F.Cu F.Paste F.Mask))
  (pad 40 smd rect (at -4.09956 -1.24968 45) (size 1.30048 0.29972) (layers F.Cu F.Paste F.Mask))
  (pad 41 smd rect (at -4.09956 -0.7493 45) (size 1.30048 0.29972) (layers F.Cu F.Paste F.Mask) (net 39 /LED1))
  (pad 42 smd rect (at -4.09956 -0.24892 45) (size 1.30048 0.29972) (layers F.Cu F.Paste F.Mask) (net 27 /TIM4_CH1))
  (pad 43 smd rect (at -4.09956 0.24892 45) (size 1.30048 0.29972) (layers F.Cu F.Paste F.Mask) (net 28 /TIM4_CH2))
  (pad 44 smd rect (at -4.09956 0.7493 45) (size 1.30048 0.29972) (layers F.Cu F.Paste F.Mask) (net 4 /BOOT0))
  (pad 9 smd rect (at 1.24968 4.09956 45) (size 0.29972 1.30048) (layers F.Cu F.Paste F.Mask) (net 1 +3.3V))
  (pad 10 smd rect (at 1.75006 4.09956 45) (size 0.29972 1.30048) (layers F.Cu F.Paste F.Mask))
  (pad 11 smd rect (at 2.25044 4.09956 45) (size 0.29972 1.30048) (layers F.Cu F.Paste F.Mask) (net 31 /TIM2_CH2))
  (pad 12 smd rect (at 2.75082 4.09956 45) (size 0.29972 1.30048) (layers F.Cu F.Paste F.Mask) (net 8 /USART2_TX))
  (pad 21 smd rect (at 4.09956 -1.24968 45) (size 1.30048 0.29972) (layers F.Cu F.Paste F.Mask) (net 40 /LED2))
  (pad 22 smd rect (at 4.09956 -1.75006 45) (size 1.30048 0.29972) (layers F.Cu F.Paste F.Mask) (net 41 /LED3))
  (pad 23 smd rect (at 4.09956 -2.25044 45) (size 1.30048 0.29972) (layers F.Cu F.Paste F.Mask) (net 2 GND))
  (pad 24 smd rect (at 4.09956 -2.75082 45) (size 1.30048 0.29972) (layers F.Cu F.Paste F.Mask) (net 1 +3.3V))
  (pad 33 smd rect (at -1.24968 -4.09956 45) (size 0.29972 1.30048) (layers F.Cu F.Paste F.Mask) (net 38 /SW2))
  (pad 34 smd rect (at -1.75006 -4.09956 45) (size 0.29972 1.30048) (layers F.Cu F.Paste F.Mask))
  (pad 35 smd rect (at -2.25044 -4.09956 45) (size 0.29972 1.30048) (layers F.Cu F.Paste F.Mask) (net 2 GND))
  (pad 36 smd rect (at -2.75082 -4.09956 45) (size 0.29972 1.30048) (layers F.Cu F.Paste F.Mask) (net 1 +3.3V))
  (pad 45 smd rect (at -4.09956 1.24968 45) (size 1.30048 0.29972) (layers F.Cu F.Paste F.Mask) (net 29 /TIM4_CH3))
  (pad 46 smd rect (at -4.09956 1.75006 45) (size 1.30048 0.29972) (layers F.Cu F.Paste F.Mask) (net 30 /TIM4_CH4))
  (pad 47 smd rect (at -4.09956 2.25044 45) (size 1.30048 0.29972) (layers F.Cu F.Paste F.Mask) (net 2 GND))
  (pad 48 smd rect (at -4.09956 2.75082 45) (size 1.30048 0.29972) (layers F.Cu F.Paste F.Mask) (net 1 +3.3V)))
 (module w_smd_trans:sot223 (layer F.Cu) (at 143.3 111.3 270)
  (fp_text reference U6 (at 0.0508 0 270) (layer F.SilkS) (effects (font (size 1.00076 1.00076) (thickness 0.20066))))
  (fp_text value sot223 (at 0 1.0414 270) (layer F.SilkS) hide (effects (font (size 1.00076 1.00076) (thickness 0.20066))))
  (pad 1 smd rect (at -2.30124 2.99974 270) (size 1.30048 1.80086) (layers F.Cu F.Paste F.Mask) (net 2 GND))
  (pad 2 smd rect (at 0 2.99974 270) (size 1.30048 1.80086) (layers F.Cu F.Paste F.Mask) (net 1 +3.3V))
  (pad 3 smd rect (at 2.30124 2.99974 270) (size 1.30048 1.80086) (layers F.Cu F.Paste F.Mask) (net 3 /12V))
  (pad 4 smd rect (at 0 -2.99974 270) (size 3.79984 1.80086) (layers F.Cu F.Paste F.Mask) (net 1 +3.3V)))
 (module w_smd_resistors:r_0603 (layer F.Cu) (at 133.8 96.45 90)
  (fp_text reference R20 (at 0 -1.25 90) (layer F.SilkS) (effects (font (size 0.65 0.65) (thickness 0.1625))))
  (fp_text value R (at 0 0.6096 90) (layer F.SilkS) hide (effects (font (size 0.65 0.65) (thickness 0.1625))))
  (pad 1 smd rect (at 0.75184 0 90) (size 0.89916 1.00076) (layers F.Cu F.Paste F.Mask) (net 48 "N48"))
  (pad 2 smd rect (at -0.75184 0 90) (size 0.89916 1.00076) (layers F.Cu F.Paste F.Mask) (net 47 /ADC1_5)))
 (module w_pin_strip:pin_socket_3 (layer F.Cu) (at 130.5 104.56 90)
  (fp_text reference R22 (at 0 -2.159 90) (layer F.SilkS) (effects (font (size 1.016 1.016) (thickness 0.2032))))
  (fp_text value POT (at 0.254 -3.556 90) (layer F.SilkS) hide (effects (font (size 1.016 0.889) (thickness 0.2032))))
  (pad 1 thru_hole rect (at -2.54 0 90) (size 1.524 2.19964) (drill 1.00076) (layers *.Cu *.Mask F.SilkS) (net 2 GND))
  (pad 2 thru_hole oval (at 0 0 90) (size 1.524 2.19964) (drill 1.00076) (layers *.Cu *.Mask F.SilkS) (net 43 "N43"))
  (pad 3 thru_hole oval (at 2.54 0 90) (size 1.524 2.19964) (drill 1.00076) (layers *.Cu *.Mask F.SilkS) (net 1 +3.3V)))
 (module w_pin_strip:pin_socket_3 (layer F.Cu) (at 130.5 94.36 90)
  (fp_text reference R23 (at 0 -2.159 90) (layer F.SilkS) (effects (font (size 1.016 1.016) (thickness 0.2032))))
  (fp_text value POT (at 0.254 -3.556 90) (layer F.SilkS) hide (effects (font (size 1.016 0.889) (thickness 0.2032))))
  (pad 1 thru_hole rect (at -2.54 0 90) (size 1.524 2.19964) (drill 1.00076) (layers *.Cu *.Mask F.SilkS) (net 2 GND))
  (pad 2 thru_hole oval (at 0 0 90) (size 1.524 2.19964) (drill 1.00076) (layers *.Cu *.Mask F.SilkS) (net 48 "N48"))
  (pad 3 thru_hole oval (at 2.54 0 90) (size 1.524 2.19964) (drill 1.00076) (layers *.Cu *.Mask F.SilkS) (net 1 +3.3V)))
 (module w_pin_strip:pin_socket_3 (layer F.Cu) (at 130.5 83.99 90)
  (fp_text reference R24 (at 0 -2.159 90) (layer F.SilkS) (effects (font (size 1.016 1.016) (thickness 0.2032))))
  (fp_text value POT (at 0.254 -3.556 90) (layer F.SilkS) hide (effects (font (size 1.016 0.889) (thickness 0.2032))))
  (pad 1 thru_hole rect (at -2.54 0 90) (size 1.524 2.19964) (drill 1.00076) (layers *.Cu *.Mask F.SilkS) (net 2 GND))
  (pad 2 thru_hole oval (at 0 0 90) (size 1.524 2.19964) (drill 1.00076) (layers *.Cu *.Mask F.SilkS) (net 45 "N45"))
  (pad 3 thru_hole oval (at 2.54 0 90) (size 1.524 2.19964) (drill 1.00076) (layers *.Cu *.Mask F.SilkS) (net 1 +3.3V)))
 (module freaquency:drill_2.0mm (layer F.Cu) (at 154.45 133.95)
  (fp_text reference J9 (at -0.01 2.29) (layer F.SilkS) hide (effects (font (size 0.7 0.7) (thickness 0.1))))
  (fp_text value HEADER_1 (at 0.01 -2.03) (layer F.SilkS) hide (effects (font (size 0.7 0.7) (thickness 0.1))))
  (pad 1 thru_hole circle (at 0 0) (size 3 3) (drill 2) (layers *.Cu *.Mask F.SilkS) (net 2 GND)))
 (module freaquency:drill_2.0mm (layer F.Cu) (at 130 134)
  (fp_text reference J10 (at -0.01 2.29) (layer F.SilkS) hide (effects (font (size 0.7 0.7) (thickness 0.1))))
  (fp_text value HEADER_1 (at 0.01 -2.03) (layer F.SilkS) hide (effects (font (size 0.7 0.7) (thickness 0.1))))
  (pad 1 thru_hole circle (at 0 0) (size 3 3) (drill 2) (layers *.Cu *.Mask F.SilkS) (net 2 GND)))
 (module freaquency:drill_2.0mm (layer F.Cu) (at 134.6 82.5)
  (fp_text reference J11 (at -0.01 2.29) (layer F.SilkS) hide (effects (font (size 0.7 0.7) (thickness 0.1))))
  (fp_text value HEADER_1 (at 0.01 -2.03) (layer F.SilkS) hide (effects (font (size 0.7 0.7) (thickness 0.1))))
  (pad 1 thru_hole circle (at 0 0) (size 3 3) (drill 2) (layers *.Cu *.Mask F.SilkS) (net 2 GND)))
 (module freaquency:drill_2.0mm (layer F.Cu) (at 167.1 87.9)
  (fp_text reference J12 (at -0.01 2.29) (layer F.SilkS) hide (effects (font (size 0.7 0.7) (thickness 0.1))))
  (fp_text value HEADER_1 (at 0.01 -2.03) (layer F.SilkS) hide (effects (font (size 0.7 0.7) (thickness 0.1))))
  (pad 1 thru_hole circle (at 0 0) (size 3 3) (drill 2) (layers *.Cu *.Mask F.SilkS) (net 2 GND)))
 (gr_line (start 169.5 79) (end 127 79) (layer Edge.Cuts) (width 0.1))
 (gr_line (start 127 137.5) (end 169.5 137.5) (layer Edge.Cuts) (width 0.1))
 (gr_line (start 127 137.5) (end 127 79) (layer Edge.Cuts) (width 0.1))
 (gr_line (start 169.5 137.5) (end 169.5 79) (layer Edge.Cuts) (width 0.1))
 (segment (start 144.531008 126.628662) (end 143.4 127.75967) (width 0.3) (layer F.Cu) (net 4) (status 400000))
 (via (at 143.4 128.2) (size 0.6) (drill 0.3) (layers F.Cu B.Cu) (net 4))
 (segment (start 143.4 127.75967) (end 143.4 128.2) (width 0.3) (layer F.Cu) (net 4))
 (segment (start 144.884831 126.982484) (end 144.099998 127.767317) (width 0.3) (layer F.Cu) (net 29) (status 400000))
 (segment (start 157.000002 124.999998) (end 157.75184 124.24816) (width 0.3) (layer F.Cu) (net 29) (status 800000))
 (segment (start 157.000002 126.257108) (end 157.000002 124.999998) (width 0.3) (layer F.Cu) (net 29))
 (segment (start 149.907108 133.350002) (end 157.000002 126.257108) (width 0.3) (layer F.Cu) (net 29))
 (segment (start 145.042892 133.350002) (end 149.907108 133.350002) (width 0.3) (layer F.Cu) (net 29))
 (segment (start 144.099998 132.407108) (end 145.042892 133.350002) (width 0.3) (layer F.Cu) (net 29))
 (segment (start 144.099998 127.767317) (end 144.099998 132.407108) (width 0.3) (layer F.Cu) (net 29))
 (segment (start 157.75184 124.24816) (end 158.25 124.24816) (width 0.3) (layer F.Cu) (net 29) (status C00000))
 (segment (start 145.238653 127.336306) (end 144.6 127.974959) (width 0.3) (layer F.Cu) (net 30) (status 400000))
 (segment (start 157.25184 120.24816) (end 158.25 120.24816) (width 0.3) (layer F.Cu) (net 30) (status 800000))
 (segment (start 156.5 121) (end 157.25184 120.24816) (width 0.3) (layer F.Cu) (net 30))
 (segment (start 156.5 126.05) (end 156.5 121) (width 0.3) (layer F.Cu) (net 30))
 (segment (start 149.7 132.85) (end 156.5 126.05) (width 0.3) (layer F.Cu) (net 30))
 (segment (start 145.25 132.85) (end 149.7 132.85) (width 0.3) (layer F.Cu) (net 30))
 (segment (start 144.6 132.2) (end 145.25 132.85) (width 0.3) (layer F.Cu) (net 30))
 (segment (start 144.6 127.974959) (end 144.6 132.2) (width 0.3) (layer F.Cu) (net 30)))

